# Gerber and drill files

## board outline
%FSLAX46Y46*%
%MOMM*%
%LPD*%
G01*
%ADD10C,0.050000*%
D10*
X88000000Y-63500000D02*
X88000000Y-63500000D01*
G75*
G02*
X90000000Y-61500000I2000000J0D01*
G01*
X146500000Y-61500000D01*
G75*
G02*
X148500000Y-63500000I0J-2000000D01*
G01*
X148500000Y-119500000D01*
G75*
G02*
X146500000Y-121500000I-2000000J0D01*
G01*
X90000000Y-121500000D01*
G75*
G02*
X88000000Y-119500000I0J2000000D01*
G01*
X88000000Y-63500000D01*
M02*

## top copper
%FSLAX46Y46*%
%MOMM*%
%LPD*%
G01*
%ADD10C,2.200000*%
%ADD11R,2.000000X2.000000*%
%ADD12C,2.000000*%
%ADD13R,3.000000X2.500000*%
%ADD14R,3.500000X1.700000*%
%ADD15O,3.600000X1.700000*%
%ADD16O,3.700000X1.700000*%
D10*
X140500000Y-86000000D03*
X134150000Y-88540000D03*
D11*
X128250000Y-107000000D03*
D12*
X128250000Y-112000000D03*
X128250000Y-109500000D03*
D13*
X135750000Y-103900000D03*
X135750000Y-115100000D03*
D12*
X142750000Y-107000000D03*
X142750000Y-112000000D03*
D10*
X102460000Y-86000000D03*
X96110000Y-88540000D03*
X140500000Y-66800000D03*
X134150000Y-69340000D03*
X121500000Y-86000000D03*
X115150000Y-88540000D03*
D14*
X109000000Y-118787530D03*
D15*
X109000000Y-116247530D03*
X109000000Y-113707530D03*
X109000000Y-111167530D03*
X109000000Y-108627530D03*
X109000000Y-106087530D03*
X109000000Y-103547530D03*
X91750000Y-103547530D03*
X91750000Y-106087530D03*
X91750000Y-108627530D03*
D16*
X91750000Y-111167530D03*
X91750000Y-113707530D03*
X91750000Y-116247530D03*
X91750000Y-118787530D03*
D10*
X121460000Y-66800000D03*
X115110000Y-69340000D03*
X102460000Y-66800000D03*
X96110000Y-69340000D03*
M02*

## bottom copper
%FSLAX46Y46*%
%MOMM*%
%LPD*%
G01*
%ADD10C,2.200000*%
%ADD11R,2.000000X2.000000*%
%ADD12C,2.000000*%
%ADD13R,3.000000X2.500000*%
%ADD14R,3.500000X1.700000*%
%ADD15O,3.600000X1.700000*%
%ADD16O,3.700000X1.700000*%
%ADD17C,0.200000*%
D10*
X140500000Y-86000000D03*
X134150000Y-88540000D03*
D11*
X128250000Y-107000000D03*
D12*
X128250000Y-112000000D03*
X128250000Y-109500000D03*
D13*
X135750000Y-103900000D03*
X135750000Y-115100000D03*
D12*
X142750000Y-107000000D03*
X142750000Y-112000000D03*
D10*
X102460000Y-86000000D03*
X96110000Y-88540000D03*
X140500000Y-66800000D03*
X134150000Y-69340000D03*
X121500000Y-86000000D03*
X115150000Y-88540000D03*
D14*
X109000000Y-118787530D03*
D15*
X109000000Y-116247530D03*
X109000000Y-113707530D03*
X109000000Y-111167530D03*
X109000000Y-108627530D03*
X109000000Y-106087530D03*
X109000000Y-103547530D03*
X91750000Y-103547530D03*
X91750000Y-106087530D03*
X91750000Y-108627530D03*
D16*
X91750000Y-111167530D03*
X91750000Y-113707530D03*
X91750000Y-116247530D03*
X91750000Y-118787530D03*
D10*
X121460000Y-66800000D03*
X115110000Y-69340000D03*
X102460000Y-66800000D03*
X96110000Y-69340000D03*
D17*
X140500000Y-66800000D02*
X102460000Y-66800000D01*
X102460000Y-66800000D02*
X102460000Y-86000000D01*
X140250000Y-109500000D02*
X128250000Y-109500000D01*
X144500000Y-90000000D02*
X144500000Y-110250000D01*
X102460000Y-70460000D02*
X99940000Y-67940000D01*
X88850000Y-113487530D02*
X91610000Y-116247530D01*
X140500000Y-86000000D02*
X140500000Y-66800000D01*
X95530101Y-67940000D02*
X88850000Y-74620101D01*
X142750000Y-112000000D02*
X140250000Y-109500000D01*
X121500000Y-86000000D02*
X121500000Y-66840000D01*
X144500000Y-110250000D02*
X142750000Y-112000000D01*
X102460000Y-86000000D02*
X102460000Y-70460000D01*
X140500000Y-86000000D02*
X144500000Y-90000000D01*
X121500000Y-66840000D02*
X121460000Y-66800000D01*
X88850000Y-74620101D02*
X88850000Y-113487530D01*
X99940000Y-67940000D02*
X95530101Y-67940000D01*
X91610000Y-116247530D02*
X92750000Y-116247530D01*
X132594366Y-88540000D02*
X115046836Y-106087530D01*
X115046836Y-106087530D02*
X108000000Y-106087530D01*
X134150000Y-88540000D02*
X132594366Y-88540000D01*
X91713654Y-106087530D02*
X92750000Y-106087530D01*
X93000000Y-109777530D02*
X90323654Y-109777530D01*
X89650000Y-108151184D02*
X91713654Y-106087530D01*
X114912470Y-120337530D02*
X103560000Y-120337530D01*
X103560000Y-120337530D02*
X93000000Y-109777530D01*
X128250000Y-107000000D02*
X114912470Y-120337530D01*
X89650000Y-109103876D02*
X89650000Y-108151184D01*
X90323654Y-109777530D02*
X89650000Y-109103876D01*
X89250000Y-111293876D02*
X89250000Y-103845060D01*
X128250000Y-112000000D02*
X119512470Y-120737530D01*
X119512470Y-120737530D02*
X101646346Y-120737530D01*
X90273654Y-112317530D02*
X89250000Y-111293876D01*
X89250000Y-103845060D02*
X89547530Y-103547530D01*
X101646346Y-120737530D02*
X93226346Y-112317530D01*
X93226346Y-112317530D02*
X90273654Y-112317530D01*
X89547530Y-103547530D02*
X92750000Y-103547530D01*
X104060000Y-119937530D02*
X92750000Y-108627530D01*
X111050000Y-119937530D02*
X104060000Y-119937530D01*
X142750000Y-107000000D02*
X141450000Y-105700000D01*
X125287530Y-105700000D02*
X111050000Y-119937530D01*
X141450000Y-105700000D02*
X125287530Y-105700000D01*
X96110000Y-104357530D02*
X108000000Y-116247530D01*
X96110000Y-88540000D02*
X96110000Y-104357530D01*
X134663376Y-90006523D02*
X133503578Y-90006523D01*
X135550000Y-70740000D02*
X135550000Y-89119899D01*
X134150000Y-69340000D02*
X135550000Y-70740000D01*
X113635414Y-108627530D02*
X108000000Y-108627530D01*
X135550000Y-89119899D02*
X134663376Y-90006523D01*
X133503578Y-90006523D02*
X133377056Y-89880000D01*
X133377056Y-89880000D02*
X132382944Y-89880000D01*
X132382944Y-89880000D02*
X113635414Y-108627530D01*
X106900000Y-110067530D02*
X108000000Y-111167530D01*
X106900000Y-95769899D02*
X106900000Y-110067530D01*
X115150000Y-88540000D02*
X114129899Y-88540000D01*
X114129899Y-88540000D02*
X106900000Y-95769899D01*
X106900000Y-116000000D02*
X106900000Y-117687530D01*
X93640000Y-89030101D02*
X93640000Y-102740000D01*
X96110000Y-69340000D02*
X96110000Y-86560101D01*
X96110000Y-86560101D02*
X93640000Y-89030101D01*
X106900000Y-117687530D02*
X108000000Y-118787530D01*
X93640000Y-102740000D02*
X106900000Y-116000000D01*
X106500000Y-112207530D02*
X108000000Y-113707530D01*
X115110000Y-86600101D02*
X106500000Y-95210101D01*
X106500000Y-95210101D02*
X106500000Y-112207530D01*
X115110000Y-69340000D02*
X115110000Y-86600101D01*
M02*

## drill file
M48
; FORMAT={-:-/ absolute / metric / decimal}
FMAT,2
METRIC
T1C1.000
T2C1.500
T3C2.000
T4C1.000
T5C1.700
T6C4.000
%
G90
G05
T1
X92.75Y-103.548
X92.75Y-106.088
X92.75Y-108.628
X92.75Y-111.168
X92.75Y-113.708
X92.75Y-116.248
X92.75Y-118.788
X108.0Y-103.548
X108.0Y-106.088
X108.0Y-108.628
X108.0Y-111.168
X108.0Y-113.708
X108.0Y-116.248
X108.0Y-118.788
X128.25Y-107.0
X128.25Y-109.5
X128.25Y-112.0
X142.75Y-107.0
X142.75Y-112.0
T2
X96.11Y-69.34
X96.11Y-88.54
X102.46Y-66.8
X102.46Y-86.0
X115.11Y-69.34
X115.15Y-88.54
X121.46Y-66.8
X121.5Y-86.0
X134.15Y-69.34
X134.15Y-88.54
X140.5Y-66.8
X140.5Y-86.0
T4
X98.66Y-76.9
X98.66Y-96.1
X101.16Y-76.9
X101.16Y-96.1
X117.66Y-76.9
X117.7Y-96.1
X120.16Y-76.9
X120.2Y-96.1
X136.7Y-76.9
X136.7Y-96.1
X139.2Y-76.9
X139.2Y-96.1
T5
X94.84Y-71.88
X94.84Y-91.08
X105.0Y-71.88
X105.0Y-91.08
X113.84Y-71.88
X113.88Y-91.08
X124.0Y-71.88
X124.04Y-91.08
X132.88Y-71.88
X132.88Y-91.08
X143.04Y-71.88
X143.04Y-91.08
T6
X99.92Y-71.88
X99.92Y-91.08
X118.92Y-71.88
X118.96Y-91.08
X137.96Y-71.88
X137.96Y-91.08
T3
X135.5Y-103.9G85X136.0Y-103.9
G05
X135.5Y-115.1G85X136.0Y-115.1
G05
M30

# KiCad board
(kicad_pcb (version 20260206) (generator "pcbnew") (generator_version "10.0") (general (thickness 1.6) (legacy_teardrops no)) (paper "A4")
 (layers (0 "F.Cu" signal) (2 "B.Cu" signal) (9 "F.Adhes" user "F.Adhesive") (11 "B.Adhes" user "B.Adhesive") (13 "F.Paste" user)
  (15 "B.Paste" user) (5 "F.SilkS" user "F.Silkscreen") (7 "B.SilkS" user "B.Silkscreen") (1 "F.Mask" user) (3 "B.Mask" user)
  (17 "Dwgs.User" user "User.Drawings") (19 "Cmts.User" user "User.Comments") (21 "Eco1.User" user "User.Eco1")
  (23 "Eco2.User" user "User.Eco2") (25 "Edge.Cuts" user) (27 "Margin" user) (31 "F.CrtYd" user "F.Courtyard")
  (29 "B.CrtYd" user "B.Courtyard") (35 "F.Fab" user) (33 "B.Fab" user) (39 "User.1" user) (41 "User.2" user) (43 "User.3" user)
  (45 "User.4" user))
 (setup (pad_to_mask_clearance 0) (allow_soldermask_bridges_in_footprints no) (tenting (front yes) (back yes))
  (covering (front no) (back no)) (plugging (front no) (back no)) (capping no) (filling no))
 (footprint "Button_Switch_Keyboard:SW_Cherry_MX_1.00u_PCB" (layer "F.Cu") (at 140.5 86)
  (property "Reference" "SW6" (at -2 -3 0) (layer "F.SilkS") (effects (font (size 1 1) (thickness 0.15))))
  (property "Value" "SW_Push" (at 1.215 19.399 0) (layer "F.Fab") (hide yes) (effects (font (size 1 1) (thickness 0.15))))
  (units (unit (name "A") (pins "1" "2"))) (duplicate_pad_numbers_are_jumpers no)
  (pad "" np_thru_hole circle (at -7.62 5.08) (size 1.7 1.7) (drill 1.7) (layers "*.Cu" "*.Mask"))
  (pad "" np_thru_hole circle (at -3.8 10.1) (size 1 1) (drill 1) (layers "*.Cu" "*.Mask"))
  (pad "" np_thru_hole circle (at -2.54 5.08) (size 4 4) (drill 4) (layers "*.Cu" "*.Mask"))
  (pad "" np_thru_hole circle (at -1.3 10.1) (size 1 1) (drill 1) (layers "*.Cu" "*.Mask"))
  (pad "" np_thru_hole circle (at 2.54 5.08) (size 1.7 1.7) (drill 1.7) (layers "*.Cu" "*.Mask"))
  (pad "1" thru_hole circle (at 0 0) (size 2.2 2.2) (drill 1.5) (layers "*.Cu" "*.Mask") (remove_unused_layers no) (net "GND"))
  (pad "2" thru_hole circle (at -6.35 2.54) (size 2.2 2.2) (drill 1.5) (layers "*.Cu" "*.Mask") (remove_unused_layers no)
   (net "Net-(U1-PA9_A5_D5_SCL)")))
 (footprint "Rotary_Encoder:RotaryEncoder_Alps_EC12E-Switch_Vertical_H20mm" (layer "F.Cu") (at 128.25 107)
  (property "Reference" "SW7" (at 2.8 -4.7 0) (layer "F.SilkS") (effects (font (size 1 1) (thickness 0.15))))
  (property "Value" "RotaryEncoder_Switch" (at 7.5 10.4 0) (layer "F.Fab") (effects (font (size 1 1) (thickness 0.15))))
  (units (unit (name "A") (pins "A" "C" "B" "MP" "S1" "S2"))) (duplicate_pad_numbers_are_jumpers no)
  (pad "A" thru_hole rect (at 0 0) (size 2 2) (drill 1) (layers "*.Cu" "*.Mask") (remove_unused_layers no) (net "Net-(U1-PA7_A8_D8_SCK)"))
  (pad "B" thru_hole circle (at 0 5) (size 2 2) (drill 1) (layers "*.Cu" "*.Mask") (remove_unused_layers no) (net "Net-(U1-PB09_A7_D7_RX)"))
  (pad "C" thru_hole circle (at 0 2.5) (size 2 2) (drill 1) (layers "*.Cu" "*.Mask") (remove_unused_layers no) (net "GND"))
  (pad "MP" thru_hole rect (at 7.5 -3.1) (size 3 2.5) (drill oval 2.5 2) (layers "*.Cu" "*.Mask") (remove_unused_layers no)
   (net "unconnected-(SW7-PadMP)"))
  (pad "MP" thru_hole rect (at 7.5 8.1) (size 3 2.5) (drill oval 2.5 2) (layers "*.Cu" "*.Mask") (remove_unused_layers no)
   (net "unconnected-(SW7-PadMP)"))
  (pad "S1" thru_hole circle (at 14.5 0) (size 2 2) (drill 1) (layers "*.Cu" "*.Mask") (remove_unused_layers no)
   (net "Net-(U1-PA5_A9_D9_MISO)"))
  (pad "S2" thru_hole circle (at 14.5 5) (size 2 2) (drill 1) (layers "*.Cu" "*.Mask") (remove_unused_layers no) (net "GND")))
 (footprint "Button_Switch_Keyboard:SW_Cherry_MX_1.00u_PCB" (layer "F.Cu") (at 102.46 86)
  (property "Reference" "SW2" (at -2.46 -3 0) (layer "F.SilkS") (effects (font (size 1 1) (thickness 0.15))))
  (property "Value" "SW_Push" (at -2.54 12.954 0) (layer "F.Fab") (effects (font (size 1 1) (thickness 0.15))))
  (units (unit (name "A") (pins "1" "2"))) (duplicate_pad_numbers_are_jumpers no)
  (pad "" np_thru_hole circle (at -7.62 5.08) (size 1.7 1.7) (drill 1.7) (layers "*.Cu" "*.Mask"))
  (pad "" np_thru_hole circle (at -3.8 10.1) (size 1 1) (drill 1) (layers "*.Cu" "*.Mask"))
  (pad "" np_thru_hole circle (at -2.54 5.08) (size 4 4) (drill 4) (layers "*.Cu" "*.Mask"))
  (pad "" np_thru_hole circle (at -1.3 10.1) (size 1 1) (drill 1) (layers "*.Cu" "*.Mask"))
  (pad "" np_thru_hole circle (at 2.54 5.08) (size 1.7 1.7) (drill 1.7) (layers "*.Cu" "*.Mask"))
  (pad "1" thru_hole circle (at 0 0) (size 2.2 2.2) (drill 1.5) (layers "*.Cu" "*.Mask") (remove_unused_layers no) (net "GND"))
  (pad "2" thru_hole circle (at -6.35 2.54) (size 2.2 2.2) (drill 1.5) (layers "*.Cu" "*.Mask") (remove_unused_layers no)
   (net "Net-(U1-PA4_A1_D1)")))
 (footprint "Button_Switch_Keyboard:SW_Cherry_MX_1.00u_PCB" (layer "F.Cu") (at 140.5 66.8)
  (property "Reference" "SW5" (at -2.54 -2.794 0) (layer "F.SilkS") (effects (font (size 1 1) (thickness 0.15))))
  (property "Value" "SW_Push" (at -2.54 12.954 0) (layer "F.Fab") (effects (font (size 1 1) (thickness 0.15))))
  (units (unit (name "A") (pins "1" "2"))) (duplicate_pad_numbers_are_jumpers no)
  (pad "" np_thru_hole circle (at -7.62 5.08) (size 1.7 1.7) (drill 1.7) (layers "*.Cu" "*.Mask"))
  (pad "" np_thru_hole circle (at -3.8 10.1) (size 1 1) (drill 1) (layers "*.Cu" "*.Mask"))
  (pad "" np_thru_hole circle (at -2.54 5.08) (size 4 4) (drill 4) (layers "*.Cu" "*.Mask"))
  (pad "" np_thru_hole circle (at -1.3 10.1) (size 1 1) (drill 1) (layers "*.Cu" "*.Mask"))
  (pad "" np_thru_hole circle (at 2.54 5.08) (size 1.7 1.7) (drill 1.7) (layers "*.Cu" "*.Mask"))
  (pad "1" thru_hole circle (at 0 0) (size 2.2 2.2) (drill 1.5) (layers "*.Cu" "*.Mask") (remove_unused_layers no) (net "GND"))
  (pad "2" thru_hole circle (at -6.35 2.54) (size 2.2 2.2) (drill 1.5) (layers "*.Cu" "*.Mask") (remove_unused_layers no)
   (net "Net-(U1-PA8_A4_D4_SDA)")))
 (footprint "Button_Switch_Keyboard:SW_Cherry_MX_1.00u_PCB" (layer "F.Cu") (at 121.5 86)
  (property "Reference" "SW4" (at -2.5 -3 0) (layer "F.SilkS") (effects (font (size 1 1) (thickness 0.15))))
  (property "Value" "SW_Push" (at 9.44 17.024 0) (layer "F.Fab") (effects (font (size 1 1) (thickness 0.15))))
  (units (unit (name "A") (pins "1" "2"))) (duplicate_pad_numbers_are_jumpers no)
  (pad "" np_thru_hole circle (at -7.62 5.08) (size 1.7 1.7) (drill 1.7) (layers "*.Cu" "*.Mask"))
  (pad "" np_thru_hole circle (at -3.8 10.1) (size 1 1) (drill 1) (layers "*.Cu" "*.Mask"))
  (pad "" np_thru_hole circle (at -2.54 5.08) (size 4 4) (drill 4) (layers "*.Cu" "*.Mask"))
  (pad "" np_thru_hole circle (at -1.3 10.1) (size 1 1) (drill 1) (layers "*.Cu" "*.Mask"))
  (pad "" np_thru_hole circle (at 2.54 5.08) (size 1.7 1.7) (drill 1.7) (layers "*.Cu" "*.Mask"))
  (pad "1" thru_hole circle (at 0 0) (size 2.2 2.2) (drill 1.5) (layers "*.Cu" "*.Mask") (remove_unused_layers no) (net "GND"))
  (pad "2" thru_hole circle (at -6.35 2.54) (size 2.2 2.2) (drill 1.5) (layers "*.Cu" "*.Mask") (remove_unused_layers no)
   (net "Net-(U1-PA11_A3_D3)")))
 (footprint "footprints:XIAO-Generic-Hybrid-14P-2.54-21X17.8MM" (layer "F.Cu") (at 100.375 111.16753 180)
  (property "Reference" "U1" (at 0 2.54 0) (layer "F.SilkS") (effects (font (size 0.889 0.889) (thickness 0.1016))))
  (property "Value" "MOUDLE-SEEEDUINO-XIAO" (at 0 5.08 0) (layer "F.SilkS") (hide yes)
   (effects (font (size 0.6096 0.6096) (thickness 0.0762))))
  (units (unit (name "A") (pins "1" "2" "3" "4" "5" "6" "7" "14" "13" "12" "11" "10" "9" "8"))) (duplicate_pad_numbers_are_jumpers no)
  (pad "1" thru_hole rect (at -7.625 -7.62 180) (size 3.5 1.7) (drill 1 (offset -1 0)) (layers "*.Cu" "*.Mask") (remove_unused_layers no)
   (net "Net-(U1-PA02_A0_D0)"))
  (pad "2" thru_hole oval (at -7.625 -5.08 180) (size 3.6 1.7) (drill 1 (offset -1 0)) (layers "*.Cu" "*.Mask") (remove_unused_layers no)
   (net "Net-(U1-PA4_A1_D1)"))
  (pad "3" thru_hole oval (at -7.625 -2.54 180) (size 3.6 1.7) (drill 1 (offset -1 0)) (layers "*.Cu" "*.Mask") (remove_unused_layers no)
   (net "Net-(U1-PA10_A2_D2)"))
  (pad "4" thru_hole oval (at -7.625 0 180) (size 3.6 1.7) (drill 1 (offset -1 0)) (layers "*.Cu" "*.Mask") (remove_unused_layers no)
   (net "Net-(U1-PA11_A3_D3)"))
  (pad "5" thru_hole oval (at -7.625 2.54 180) (size 3.6 1.7) (drill 1 (offset -1 0)) (layers "*.Cu" "*.Mask") (remove_unused_layers no)
   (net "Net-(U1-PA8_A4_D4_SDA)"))
  (pad "6" thru_hole oval (at -7.625 5.08) (size 3.6 1.7) (drill 1 (offset 1 0)) (layers "*.Cu" "*.Mask") (remove_unused_layers no)
   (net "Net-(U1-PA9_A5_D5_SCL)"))
  (pad "7" thru_hole oval (at -7.625 7.62 180) (size 3.6 1.7) (drill 1 (offset -1 0)) (layers "*.Cu" "*.Mask") (remove_unused_layers no)
   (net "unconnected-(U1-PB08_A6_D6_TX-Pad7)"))
  (pad "8" thru_hole oval (at 7.625 7.62 180) (size 3.6 1.7) (drill 1 (offset 1 0)) (layers "*.Cu" "*.Mask") (remove_unused_layers no)
   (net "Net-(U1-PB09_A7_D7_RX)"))
  (pad "9" thru_hole oval (at 7.625 5.08 180) (size 3.6 1.7) (drill 1 (offset 1 0)) (layers "*.Cu" "*.Mask") (remove_unused_layers no)
   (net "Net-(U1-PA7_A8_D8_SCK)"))
  (pad "10" thru_hole oval (at 7.625 2.54 180) (size 3.6 1.7) (drill 1 (offset 1 0)) (layers "*.Cu" "*.Mask") (remove_unused_layers no)
   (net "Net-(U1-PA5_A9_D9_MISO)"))
  (pad "11" thru_hole oval (at 7.625 0 180) (size 3.7 1.7) (drill 1 (offset 1 0)) (layers "*.Cu" "*.Mask") (remove_unused_layers no)
   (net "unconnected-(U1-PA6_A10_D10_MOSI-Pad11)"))
  (pad "12" thru_hole oval (at 7.625 -2.54 180) (size 3.7 1.7) (drill 1 (offset 1 0)) (layers "*.Cu" "*.Mask") (remove_unused_layers no)
   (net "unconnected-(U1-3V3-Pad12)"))
  (pad "13" thru_hole oval (at 7.625 -5.08 180) (size 3.7 1.7) (drill 1 (offset 1 0)) (layers "*.Cu" "*.Mask") (remove_unused_layers no)
   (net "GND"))
  (pad "14" thru_hole oval (at 7.625 -7.62 180) (size 3.7 1.7) (drill 1 (offset 1 0)) (layers "*.Cu" "*.Mask") (remove_unused_layers no)
   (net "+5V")))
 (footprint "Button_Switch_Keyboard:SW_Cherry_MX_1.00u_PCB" (layer "F.Cu") (at 121.46 66.8)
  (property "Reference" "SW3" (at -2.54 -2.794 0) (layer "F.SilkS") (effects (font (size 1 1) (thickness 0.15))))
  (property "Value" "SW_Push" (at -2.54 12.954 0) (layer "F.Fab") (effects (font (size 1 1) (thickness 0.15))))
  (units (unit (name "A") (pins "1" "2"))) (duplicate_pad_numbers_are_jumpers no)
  (pad "" np_thru_hole circle (at -7.62 5.08) (size 1.7 1.7) (drill 1.7) (layers "*.Cu" "*.Mask"))
  (pad "" np_thru_hole circle (at -3.8 10.1) (size 1 1) (drill 1) (layers "*.Cu" "*.Mask"))
  (pad "" np_thru_hole circle (at -2.54 5.08) (size 4 4) (drill 4) (layers "*.Cu" "*.Mask"))
  (pad "" np_thru_hole circle (at -1.3 10.1) (size 1 1) (drill 1) (layers "*.Cu" "*.Mask"))
  (pad "" np_thru_hole circle (at 2.54 5.08) (size 1.7 1.7) (drill 1.7) (layers "*.Cu" "*.Mask"))
  (pad "1" thru_hole circle (at 0 0) (size 2.2 2.2) (drill 1.5) (layers "*.Cu" "*.Mask") (remove_unused_layers no) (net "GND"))
  (pad "2" thru_hole circle (at -6.35 2.54) (size 2.2 2.2) (drill 1.5) (layers "*.Cu" "*.Mask") (remove_unused_layers no)
   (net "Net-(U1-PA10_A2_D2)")))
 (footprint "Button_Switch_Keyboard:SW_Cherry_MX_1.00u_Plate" (layer "F.Cu") (at 102.46 66.8)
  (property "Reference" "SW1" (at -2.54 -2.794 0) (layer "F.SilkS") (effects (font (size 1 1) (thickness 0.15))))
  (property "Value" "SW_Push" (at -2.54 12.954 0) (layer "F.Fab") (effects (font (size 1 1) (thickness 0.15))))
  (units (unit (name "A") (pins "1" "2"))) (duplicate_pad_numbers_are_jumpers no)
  (pad "" np_thru_hole circle (at -7.62 5.08) (size 1.7 1.7) (drill 1.7) (layers "*.Cu" "*.Mask"))
  (pad "" np_thru_hole circle (at -3.8 10.1) (size 1 1) (drill 1) (layers "*.Cu" "*.Mask"))
  (pad "" np_thru_hole circle (at -2.54 5.08) (size 4 4) (drill 4) (layers "*.Cu" "*.Mask"))
  (pad "" np_thru_hole circle (at -1.3 10.1) (size 1 1) (drill 1) (layers "*.Cu" "*.Mask"))
  (pad "" np_thru_hole circle (at 2.54 5.08) (size 1.7 1.7) (drill 1.7) (layers "*.Cu" "*.Mask"))
  (pad "1" thru_hole circle (at 0 0) (size 2.2 2.2) (drill 1.5) (layers "*.Cu" "*.Mask") (remove_unused_layers no) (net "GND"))
  (pad "2" thru_hole circle (at -6.35 2.54) (size 2.2 2.2) (drill 1.5) (layers "*.Cu" "*.Mask") (remove_unused_layers no)
   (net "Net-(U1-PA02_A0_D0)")))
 (gr_rect (start 88 61.5) (end 148.5 121.5) (radius 2) (stroke (width 0.05) (type default)) (fill no) (layer "Edge.Cuts"))
 (segment (start 140.5 66.8) (end 102.46 66.8) (width 0.2) (layer "B.Cu") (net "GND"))
 (segment (start 102.46 66.8) (end 102.46 86) (width 0.2) (layer "B.Cu") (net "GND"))
 (segment (start 140.25 109.5) (end 128.25 109.5) (width 0.2) (layer "B.Cu") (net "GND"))
 (segment (start 144.5 90) (end 144.5 110.25) (width 0.2) (layer "B.Cu") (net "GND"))
 (segment (start 102.46 70.46) (end 99.94 67.94) (width 0.2) (layer "B.Cu") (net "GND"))
 (segment (start 88.85 113.48753) (end 91.61 116.24753) (width 0.2) (layer "B.Cu") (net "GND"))
 (segment (start 140.5 86) (end 140.5 66.8) (width 0.2) (layer "B.Cu") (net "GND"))
 (segment (start 95.530101 67.94) (end 88.85 74.620101) (width 0.2) (layer "B.Cu") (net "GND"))
 (segment (start 142.75 112) (end 140.25 109.5) (width 0.2) (layer "B.Cu") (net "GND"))
 (segment (start 121.5 86) (end 121.5 66.84) (width 0.2) (layer "B.Cu") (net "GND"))
 (segment (start 144.5 110.25) (end 142.75 112) (width 0.2) (layer "B.Cu") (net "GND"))
 (segment (start 102.46 86) (end 102.46 70.46) (width 0.2) (layer "B.Cu") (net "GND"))
 (segment (start 140.5 86) (end 144.5 90) (width 0.2) (layer "B.Cu") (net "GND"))
 (segment (start 121.5 66.84) (end 121.46 66.8) (width 0.2) (layer "B.Cu") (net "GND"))
 (segment (start 88.85 74.620101) (end 88.85 113.48753) (width 0.2) (layer "B.Cu") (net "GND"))
 (segment (start 99.94 67.94) (end 95.530101 67.94) (width 0.2) (layer "B.Cu") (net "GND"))
 (segment (start 91.61 116.24753) (end 92.75 116.24753) (width 0.2) (layer "B.Cu") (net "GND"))
 (segment (start 132.594366 88.54) (end 115.046836 106.08753) (width 0.2) (layer "B.Cu") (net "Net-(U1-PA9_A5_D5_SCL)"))
 (segment (start 115.046836 106.08753) (end 108 106.08753) (width 0.2) (layer "B.Cu") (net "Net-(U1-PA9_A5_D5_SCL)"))
 (segment (start 134.15 88.54) (end 132.594366 88.54) (width 0.2) (layer "B.Cu") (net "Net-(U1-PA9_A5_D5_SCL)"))
 (segment (start 91.713654 106.08753) (end 92.75 106.08753) (width 0.2) (layer "B.Cu") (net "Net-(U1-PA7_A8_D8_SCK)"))
 (segment (start 93 109.77753) (end 90.323654 109.77753) (width 0.2) (layer "B.Cu") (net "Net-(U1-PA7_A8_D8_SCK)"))
 (segment (start 89.65 108.151184) (end 91.713654 106.08753) (width 0.2) (layer "B.Cu") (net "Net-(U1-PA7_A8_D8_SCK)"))
 (segment (start 114.91247 120.33753) (end 103.56 120.33753) (width 0.2) (layer "B.Cu") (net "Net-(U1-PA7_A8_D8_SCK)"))
 (segment (start 103.56 120.33753) (end 93 109.77753) (width 0.2) (layer "B.Cu") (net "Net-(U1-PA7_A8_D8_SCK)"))
 (segment (start 128.25 107) (end 114.91247 120.33753) (width 0.2) (layer "B.Cu") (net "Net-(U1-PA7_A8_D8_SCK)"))
 (segment (start 89.65 109.103876) (end 89.65 108.151184) (width 0.2) (layer "B.Cu") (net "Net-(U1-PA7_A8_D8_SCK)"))
 (segment (start 90.323654 109.77753) (end 89.65 109.103876) (width 0.2) (layer "B.Cu") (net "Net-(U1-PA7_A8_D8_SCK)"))
 (segment (start 89.25 111.293876) (end 89.25 103.84506) (width 0.2) (layer "B.Cu") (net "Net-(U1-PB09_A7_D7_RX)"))
 (segment (start 128.25 112) (end 119.51247 120.73753) (width 0.2) (layer "B.Cu") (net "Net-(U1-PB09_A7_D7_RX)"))
 (segment (start 119.51247 120.73753) (end 101.646346 120.73753) (width 0.2) (layer "B.Cu") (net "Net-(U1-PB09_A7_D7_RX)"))
 (segment (start 90.273654 112.31753) (end 89.25 111.293876) (width 0.2) (layer "B.Cu") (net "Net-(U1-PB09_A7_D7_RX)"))
 (segment (start 89.25 103.84506) (end 89.54753 103.54753) (width 0.2) (layer "B.Cu") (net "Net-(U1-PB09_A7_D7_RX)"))
 (segment (start 101.646346 120.73753) (end 93.226346 112.31753) (width 0.2) (layer "B.Cu") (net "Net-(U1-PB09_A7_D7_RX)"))
 (segment (start 93.226346 112.31753) (end 90.273654 112.31753) (width 0.2) (layer "B.Cu") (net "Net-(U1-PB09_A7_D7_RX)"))
 (segment (start 89.54753 103.54753) (end 92.75 103.54753) (width 0.2) (layer "B.Cu") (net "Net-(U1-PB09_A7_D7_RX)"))
 (segment (start 104.06 119.93753) (end 92.75 108.62753) (width 0.2) (layer "B.Cu") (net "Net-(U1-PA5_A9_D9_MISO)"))
 (segment (start 111.05 119.93753) (end 104.06 119.93753) (width 0.2) (layer "B.Cu") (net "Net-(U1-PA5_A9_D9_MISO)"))
 (segment (start 142.75 107) (end 141.45 105.7) (width 0.2) (layer "B.Cu") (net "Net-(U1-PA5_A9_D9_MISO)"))
 (segment (start 125.28753 105.7) (end 111.05 119.93753) (width 0.2) (layer "B.Cu") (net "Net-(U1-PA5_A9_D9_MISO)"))
 (segment (start 141.45 105.7) (end 125.28753 105.7) (width 0.2) (layer "B.Cu") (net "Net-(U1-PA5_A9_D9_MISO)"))
 (segment (start 96.11 104.35753) (end 108 116.24753) (width 0.2) (layer "B.Cu") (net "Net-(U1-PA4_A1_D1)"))
 (segment (start 96.11 88.54) (end 96.11 104.35753) (width 0.2) (layer "B.Cu") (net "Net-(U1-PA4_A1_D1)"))
 (segment (start 134.663376 90.006523) (end 133.503578 90.006523) (width 0.2) (layer "B.Cu") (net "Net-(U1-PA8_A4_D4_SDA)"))
 (segment (start 135.55 70.74) (end 135.55 89.119899) (width 0.2) (layer "B.Cu") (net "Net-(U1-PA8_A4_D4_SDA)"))
 (segment (start 134.15 69.34) (end 135.55 70.74) (width 0.2) (layer "B.Cu") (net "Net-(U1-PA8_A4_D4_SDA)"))
 (segment (start 113.635414 108.62753) (end 108 108.62753) (width 0.2) (layer "B.Cu") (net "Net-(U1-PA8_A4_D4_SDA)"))
 (segment (start 135.55 89.119899) (end 134.663376 90.006523) (width 0.2) (layer "B.Cu") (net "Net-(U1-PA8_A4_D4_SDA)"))
 (segment (start 133.503578 90.006523) (end 133.377056 89.88) (width 0.2) (layer "B.Cu") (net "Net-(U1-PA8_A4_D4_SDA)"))
 (segment (start 133.377056 89.88) (end 132.382944 89.88) (width 0.2) (layer "B.Cu") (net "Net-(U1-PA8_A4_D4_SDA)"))
 (segment (start 132.382944 89.88) (end 113.635414 108.62753) (width 0.2) (layer "B.Cu") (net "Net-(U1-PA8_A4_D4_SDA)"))
 (segment (start 106.9 110.06753) (end 108 111.16753) (width 0.2) (layer "B.Cu") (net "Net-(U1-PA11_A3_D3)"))
 (segment (start 106.9 95.769899) (end 106.9 110.06753) (width 0.2) (layer "B.Cu") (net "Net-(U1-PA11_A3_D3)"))
 (segment (start 115.15 88.54) (end 114.129899 88.54) (width 0.2) (layer "B.Cu") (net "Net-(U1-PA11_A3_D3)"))
 (segment (start 114.129899 88.54) (end 106.9 95.769899) (width 0.2) (layer "B.Cu") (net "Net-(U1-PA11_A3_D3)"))
 (segment (start 106.9 116) (end 106.9 117.68753) (width 0.2) (layer "B.Cu") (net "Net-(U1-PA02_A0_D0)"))
 (segment (start 93.64 89.030101) (end 93.64 102.74) (width 0.2) (layer "B.Cu") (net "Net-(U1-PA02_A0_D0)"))
 (segment (start 96.11 69.34) (end 96.11 86.560101) (width 0.2) (layer "B.Cu") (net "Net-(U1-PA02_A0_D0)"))
 (segment (start 96.11 86.560101) (end 93.64 89.030101) (width 0.2) (layer "B.Cu") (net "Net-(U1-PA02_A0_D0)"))
 (segment (start 106.9 117.68753) (end 108 118.78753) (width 0.2) (layer "B.Cu") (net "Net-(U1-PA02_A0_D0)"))
 (segment (start 93.64 102.74) (end 106.9 116) (width 0.2) (layer "B.Cu") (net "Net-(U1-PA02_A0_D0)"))
 (segment (start 106.5 112.20753) (end 108 113.70753) (width 0.2) (layer "B.Cu") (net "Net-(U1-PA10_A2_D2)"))
 (segment (start 115.11 86.600101) (end 106.5 95.210101) (width 0.2) (layer "B.Cu") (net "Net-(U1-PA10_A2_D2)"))
 (segment (start 106.5 95.210101) (end 106.5 112.20753) (width 0.2) (layer "B.Cu") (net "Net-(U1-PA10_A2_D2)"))
 (segment (start 115.11 69.34) (end 115.11 86.600101) (width 0.2) (layer "B.Cu") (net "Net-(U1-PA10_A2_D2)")))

